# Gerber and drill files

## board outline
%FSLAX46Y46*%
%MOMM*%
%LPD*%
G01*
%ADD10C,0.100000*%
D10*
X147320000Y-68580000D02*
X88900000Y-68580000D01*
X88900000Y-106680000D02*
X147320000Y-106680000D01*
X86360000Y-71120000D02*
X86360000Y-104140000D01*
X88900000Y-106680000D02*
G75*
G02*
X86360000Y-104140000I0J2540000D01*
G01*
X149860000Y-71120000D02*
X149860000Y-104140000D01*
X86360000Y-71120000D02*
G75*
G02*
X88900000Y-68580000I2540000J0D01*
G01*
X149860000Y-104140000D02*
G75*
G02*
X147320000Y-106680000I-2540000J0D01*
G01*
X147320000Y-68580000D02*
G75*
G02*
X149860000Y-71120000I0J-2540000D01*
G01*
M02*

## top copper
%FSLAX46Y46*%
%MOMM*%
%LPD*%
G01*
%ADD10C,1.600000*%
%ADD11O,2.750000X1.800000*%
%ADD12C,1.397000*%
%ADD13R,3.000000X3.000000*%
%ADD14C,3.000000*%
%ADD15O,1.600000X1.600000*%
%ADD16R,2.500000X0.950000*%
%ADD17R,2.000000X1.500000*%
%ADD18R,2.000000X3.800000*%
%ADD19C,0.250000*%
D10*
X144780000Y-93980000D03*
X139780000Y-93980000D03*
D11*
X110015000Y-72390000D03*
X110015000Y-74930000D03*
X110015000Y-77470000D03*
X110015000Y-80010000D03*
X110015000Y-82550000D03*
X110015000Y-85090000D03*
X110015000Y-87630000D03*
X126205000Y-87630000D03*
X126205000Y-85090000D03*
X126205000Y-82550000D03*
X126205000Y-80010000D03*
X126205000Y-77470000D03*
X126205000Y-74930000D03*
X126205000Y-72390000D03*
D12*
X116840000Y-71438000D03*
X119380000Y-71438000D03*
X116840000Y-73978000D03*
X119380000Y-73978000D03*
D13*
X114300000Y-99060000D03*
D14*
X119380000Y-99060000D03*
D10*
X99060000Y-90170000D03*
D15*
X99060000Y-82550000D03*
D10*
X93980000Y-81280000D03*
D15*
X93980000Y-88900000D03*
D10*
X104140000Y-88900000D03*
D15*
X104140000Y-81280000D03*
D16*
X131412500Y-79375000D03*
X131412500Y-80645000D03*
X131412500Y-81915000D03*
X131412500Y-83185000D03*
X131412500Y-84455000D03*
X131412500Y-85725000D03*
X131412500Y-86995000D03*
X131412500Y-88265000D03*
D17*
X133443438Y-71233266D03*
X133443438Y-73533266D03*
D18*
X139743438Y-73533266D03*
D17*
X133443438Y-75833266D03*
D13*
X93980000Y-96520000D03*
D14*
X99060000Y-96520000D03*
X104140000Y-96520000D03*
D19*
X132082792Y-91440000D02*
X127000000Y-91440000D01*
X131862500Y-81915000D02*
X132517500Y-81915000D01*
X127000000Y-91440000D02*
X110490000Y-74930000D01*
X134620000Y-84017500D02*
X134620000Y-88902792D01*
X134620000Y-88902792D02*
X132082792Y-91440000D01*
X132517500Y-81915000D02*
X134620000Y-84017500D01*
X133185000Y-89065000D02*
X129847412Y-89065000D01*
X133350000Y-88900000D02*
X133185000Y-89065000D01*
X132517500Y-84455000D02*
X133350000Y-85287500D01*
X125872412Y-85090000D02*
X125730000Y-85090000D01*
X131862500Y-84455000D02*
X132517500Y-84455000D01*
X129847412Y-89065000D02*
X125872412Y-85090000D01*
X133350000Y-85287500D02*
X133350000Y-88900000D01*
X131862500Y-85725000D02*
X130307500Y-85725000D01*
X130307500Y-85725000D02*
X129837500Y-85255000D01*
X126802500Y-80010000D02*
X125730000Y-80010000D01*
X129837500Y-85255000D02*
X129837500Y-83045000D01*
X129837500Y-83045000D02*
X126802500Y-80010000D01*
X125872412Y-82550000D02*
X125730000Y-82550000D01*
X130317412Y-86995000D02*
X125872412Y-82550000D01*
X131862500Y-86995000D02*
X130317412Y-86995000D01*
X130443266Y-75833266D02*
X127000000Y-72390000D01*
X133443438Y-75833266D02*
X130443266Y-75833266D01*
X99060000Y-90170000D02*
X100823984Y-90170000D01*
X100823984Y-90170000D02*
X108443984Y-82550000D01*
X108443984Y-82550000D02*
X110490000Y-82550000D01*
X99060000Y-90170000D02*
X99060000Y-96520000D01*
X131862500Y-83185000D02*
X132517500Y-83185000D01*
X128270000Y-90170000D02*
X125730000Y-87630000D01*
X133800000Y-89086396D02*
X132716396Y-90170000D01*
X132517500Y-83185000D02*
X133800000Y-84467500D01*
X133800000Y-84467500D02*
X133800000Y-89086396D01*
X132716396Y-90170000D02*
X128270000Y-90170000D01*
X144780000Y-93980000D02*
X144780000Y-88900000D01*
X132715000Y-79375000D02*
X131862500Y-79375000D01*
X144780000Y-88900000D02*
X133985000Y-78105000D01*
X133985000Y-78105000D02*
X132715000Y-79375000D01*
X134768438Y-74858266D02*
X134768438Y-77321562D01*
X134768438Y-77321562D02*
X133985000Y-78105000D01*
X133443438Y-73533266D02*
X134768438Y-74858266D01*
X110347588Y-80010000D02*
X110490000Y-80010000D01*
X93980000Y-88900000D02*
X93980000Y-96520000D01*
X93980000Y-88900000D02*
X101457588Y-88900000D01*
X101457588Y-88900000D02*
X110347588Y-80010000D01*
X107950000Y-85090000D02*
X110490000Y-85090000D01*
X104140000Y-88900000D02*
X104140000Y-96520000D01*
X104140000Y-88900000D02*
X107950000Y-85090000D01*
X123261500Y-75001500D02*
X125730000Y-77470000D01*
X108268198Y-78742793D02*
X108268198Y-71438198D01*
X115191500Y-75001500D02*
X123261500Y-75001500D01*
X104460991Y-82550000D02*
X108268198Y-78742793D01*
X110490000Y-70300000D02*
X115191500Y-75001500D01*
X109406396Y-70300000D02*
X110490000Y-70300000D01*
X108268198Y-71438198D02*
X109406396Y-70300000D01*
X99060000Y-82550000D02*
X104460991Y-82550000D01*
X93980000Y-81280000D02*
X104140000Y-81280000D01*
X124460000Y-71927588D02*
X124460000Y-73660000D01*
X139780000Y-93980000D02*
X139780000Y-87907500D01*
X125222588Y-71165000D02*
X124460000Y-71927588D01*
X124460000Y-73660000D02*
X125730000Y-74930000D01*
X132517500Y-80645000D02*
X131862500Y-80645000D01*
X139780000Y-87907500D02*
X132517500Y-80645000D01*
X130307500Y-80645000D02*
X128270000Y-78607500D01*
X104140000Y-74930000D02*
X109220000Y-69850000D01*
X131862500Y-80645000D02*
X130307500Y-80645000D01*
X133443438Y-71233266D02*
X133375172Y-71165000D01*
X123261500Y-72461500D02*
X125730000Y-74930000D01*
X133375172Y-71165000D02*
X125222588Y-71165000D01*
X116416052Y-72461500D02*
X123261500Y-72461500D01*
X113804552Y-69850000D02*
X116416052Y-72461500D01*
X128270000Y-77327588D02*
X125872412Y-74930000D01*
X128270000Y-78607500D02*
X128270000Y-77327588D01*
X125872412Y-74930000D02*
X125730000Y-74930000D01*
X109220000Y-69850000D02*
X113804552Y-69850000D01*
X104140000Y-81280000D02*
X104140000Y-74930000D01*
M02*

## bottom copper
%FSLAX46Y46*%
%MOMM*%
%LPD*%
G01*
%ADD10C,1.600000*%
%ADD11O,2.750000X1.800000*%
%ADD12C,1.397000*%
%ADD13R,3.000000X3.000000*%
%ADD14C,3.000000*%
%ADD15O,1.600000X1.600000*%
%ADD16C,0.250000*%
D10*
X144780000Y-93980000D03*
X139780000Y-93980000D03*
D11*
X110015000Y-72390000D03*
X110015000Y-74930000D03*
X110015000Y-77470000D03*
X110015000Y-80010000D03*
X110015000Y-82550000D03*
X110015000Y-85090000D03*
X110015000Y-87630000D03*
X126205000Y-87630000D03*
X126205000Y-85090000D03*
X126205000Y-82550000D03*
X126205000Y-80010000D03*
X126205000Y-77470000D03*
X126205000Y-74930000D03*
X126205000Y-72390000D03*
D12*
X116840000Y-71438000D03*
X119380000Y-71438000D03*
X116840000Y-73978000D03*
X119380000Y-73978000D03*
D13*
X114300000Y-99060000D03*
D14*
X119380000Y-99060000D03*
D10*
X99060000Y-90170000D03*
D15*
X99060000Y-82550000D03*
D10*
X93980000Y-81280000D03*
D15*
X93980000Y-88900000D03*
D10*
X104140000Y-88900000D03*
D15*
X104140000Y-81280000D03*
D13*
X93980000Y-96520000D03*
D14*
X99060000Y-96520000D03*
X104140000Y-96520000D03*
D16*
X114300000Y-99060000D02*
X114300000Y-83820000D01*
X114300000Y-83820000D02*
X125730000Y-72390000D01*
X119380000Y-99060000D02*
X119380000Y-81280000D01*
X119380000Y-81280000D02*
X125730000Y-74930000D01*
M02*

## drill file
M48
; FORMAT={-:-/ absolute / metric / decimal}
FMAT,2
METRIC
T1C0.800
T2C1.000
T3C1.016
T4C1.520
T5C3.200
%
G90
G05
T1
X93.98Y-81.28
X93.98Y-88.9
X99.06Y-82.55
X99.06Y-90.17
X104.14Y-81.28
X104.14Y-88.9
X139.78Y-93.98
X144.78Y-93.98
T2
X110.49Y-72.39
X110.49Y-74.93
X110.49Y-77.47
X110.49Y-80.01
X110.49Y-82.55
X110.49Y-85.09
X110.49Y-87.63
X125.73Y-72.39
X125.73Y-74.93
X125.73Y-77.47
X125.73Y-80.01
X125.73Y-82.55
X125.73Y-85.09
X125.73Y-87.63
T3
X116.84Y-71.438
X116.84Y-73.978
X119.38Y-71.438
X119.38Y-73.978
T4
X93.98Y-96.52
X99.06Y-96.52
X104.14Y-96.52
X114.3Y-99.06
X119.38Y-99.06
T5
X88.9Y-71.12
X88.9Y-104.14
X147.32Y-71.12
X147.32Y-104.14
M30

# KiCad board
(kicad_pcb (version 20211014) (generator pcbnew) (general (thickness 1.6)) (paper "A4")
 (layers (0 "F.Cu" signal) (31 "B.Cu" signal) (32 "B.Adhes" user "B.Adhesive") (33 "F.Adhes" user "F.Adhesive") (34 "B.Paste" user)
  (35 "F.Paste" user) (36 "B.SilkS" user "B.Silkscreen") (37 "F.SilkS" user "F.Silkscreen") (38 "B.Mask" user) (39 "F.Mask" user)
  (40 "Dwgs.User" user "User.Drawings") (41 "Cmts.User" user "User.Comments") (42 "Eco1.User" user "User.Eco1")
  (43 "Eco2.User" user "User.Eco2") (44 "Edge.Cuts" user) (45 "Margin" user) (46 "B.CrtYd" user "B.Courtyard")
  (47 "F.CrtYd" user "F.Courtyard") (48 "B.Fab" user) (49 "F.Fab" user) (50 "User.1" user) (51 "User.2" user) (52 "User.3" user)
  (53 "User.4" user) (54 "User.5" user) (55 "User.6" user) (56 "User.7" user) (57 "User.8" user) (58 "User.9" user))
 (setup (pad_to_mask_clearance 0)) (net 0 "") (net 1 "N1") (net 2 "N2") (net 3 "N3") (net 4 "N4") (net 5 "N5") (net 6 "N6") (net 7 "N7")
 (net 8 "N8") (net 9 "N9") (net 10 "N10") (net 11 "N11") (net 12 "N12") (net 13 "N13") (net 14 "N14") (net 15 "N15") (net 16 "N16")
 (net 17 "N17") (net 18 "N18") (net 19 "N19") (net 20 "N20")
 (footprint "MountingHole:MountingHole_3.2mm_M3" (layer "F.Cu") (at 147.32 104.14)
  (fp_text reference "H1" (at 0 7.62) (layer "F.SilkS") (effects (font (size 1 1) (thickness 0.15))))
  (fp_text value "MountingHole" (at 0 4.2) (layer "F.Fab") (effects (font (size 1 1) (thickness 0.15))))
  (pad "" np_thru_hole circle (at 0 0) (size 3.2 3.2) (drill 3.2) (layers *.Cu *.Mask)))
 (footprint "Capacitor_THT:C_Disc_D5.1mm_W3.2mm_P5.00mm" (layer "F.Cu") (at 144.78 93.98 180)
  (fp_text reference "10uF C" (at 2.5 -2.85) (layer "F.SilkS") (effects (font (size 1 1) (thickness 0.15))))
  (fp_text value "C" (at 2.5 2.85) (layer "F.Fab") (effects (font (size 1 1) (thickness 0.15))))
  (pad "1" thru_hole circle (at 0 0 180) (size 1.6 1.6) (drill 0.8) (layers *.Cu *.Mask) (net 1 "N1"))
  (pad "2" thru_hole circle (at 5 0 180) (size 1.6 1.6) (drill 0.8) (layers *.Cu *.Mask) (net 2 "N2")))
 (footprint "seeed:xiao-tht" (layer "F.Cu") (at 118.11 80.01)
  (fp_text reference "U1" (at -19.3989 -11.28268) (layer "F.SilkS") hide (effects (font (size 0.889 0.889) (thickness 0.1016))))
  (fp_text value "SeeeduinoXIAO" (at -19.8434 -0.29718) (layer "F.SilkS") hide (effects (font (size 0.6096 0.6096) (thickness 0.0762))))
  (pad "1" thru_hole oval (at -7.62 -7.62) (size 2.75 1.8) (drill 1 (offset -0.475 0)) (layers *.Cu *.Mask) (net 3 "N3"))
  (pad "2" thru_hole oval (at -7.62 -5.08) (size 2.75 1.8) (drill 1 (offset -0.475 0)) (layers *.Cu *.Mask) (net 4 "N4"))
  (pad "3" thru_hole oval (at -7.62 -2.54) (size 2.75 1.8) (drill 1 (offset -0.475 0)) (layers *.Cu *.Mask) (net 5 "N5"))
  (pad "4" thru_hole oval (at -7.62 0) (size 2.75 1.8) (drill 1 (offset -0.475 0)) (layers *.Cu *.Mask) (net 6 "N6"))
  (pad "5" thru_hole oval (at -7.62 2.54) (size 2.75 1.8) (drill 1 (offset -0.475 0)) (layers *.Cu *.Mask) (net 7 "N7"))
  (pad "6" thru_hole oval (at -7.62 5.08) (size 2.75 1.8) (drill 1 (offset -0.475 0)) (layers *.Cu *.Mask) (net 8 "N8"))
  (pad "7" thru_hole oval (at -7.62 7.62) (size 2.75 1.8) (drill 1 (offset -0.475 0)) (layers *.Cu *.Mask) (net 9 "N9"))
  (pad "8" thru_hole oval (at 7.62 7.62 180) (size 2.75 1.8) (drill 1 (offset -0.475 0)) (layers *.Cu *.Mask) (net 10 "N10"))
  (pad "9" thru_hole oval (at 7.62 5.08 180) (size 2.75 1.8) (drill 1 (offset -0.475 0)) (layers *.Cu *.Mask) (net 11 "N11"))
  (pad "10" thru_hole oval (at 7.62 2.54 180) (size 2.75 1.8) (drill 1 (offset -0.475 0)) (layers *.Cu *.Mask) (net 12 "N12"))
  (pad "11" thru_hole oval (at 7.62 0 180) (size 2.75 1.8) (drill 1 (offset -0.475 0)) (layers *.Cu *.Mask) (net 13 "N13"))
  (pad "12" thru_hole oval (at 7.62 -2.54 180) (size 2.75 1.8) (drill 1 (offset -0.475 0)) (layers *.Cu *.Mask) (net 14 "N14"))
  (pad "13" thru_hole oval (at 7.62 -5.08 180) (size 2.75 1.8) (drill 1 (offset -0.475 0)) (layers *.Cu *.Mask) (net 2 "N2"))
  (pad "14" thru_hole oval (at 7.62 -7.62 180) (size 2.75 1.8) (drill 1 (offset -0.475 0)) (layers *.Cu *.Mask) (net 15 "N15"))
  (pad "15" thru_hole circle (at -1.27 -8.572 90) (size 1.397 1.397) (drill 1.016) (layers *.Cu *.Mask) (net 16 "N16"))
  (pad "16" thru_hole circle (at 1.27 -8.572 90) (size 1.397 1.397) (drill 1.016) (layers *.Cu *.Mask) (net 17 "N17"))
  (pad "17" thru_hole circle (at -1.27 -6.032 90) (size 1.397 1.397) (drill 1.016) (layers *.Cu *.Mask) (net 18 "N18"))
  (pad "18" thru_hole circle (at 1.27 -6.032 90) (size 1.397 1.397) (drill 1.016) (layers *.Cu *.Mask) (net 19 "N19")))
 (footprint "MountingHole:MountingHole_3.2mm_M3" (layer "F.Cu") (at 88.9 104.14)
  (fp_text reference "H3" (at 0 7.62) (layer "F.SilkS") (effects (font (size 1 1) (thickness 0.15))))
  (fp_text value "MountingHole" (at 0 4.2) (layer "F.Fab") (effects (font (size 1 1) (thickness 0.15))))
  (pad "" np_thru_hole circle (at 0 0) (size 3.2 3.2) (drill 3.2) (layers *.Cu *.Mask)))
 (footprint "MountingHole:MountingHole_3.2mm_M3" (layer "F.Cu") (at 147.32 71.12)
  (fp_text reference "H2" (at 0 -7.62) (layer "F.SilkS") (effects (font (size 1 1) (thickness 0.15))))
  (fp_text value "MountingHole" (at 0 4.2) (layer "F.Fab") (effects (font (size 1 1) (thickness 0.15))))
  (pad "" np_thru_hole circle (at 0 0) (size 3.2 3.2) (drill 3.2) (layers *.Cu *.Mask)))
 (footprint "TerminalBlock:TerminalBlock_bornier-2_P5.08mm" (layer "F.Cu") (at 114.3 99.06)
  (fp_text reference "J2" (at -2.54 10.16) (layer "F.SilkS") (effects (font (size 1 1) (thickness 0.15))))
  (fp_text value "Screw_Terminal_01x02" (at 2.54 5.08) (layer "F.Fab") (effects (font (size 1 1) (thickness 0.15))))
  (pad "1" thru_hole rect (at 0 0) (size 3 3) (drill 1.52) (layers *.Cu *.Mask) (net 15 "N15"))
  (pad "2" thru_hole circle (at 5.08 0) (size 3 3) (drill 1.52) (layers *.Cu *.Mask) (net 2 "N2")))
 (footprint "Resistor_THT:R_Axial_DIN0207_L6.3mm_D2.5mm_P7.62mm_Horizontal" (layer "F.Cu") (at 99.06 90.17 90)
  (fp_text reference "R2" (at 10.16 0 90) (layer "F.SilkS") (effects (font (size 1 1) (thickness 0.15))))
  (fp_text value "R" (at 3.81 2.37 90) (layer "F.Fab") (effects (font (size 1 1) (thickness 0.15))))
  (pad "1" thru_hole circle (at 0 0 90) (size 1.6 1.6) (drill 0.8) (layers *.Cu *.Mask) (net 7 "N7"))
  (pad "2" thru_hole oval (at 7.62 0 90) (size 1.6 1.6) (drill 0.8) (layers *.Cu *.Mask) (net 14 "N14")))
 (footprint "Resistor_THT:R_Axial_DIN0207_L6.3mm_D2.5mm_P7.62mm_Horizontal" (layer "F.Cu") (at 93.98 81.28 -90)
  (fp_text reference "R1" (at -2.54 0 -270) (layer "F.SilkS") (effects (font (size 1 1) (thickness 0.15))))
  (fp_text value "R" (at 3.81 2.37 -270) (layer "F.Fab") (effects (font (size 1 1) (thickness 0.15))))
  (pad "1" thru_hole circle (at 0 0 270) (size 1.6 1.6) (drill 0.8) (layers *.Cu *.Mask) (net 2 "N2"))
  (pad "2" thru_hole oval (at 7.62 0 270) (size 1.6 1.6) (drill 0.8) (layers *.Cu *.Mask) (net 6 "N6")))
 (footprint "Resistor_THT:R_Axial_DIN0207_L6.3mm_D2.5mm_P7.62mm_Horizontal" (layer "F.Cu") (at 104.14 88.9 90)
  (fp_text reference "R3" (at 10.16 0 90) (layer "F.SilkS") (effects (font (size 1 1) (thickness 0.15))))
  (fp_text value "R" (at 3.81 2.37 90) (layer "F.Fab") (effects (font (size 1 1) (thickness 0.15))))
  (pad "1" thru_hole circle (at 0 0 90) (size 1.6 1.6) (drill 0.8) (layers *.Cu *.Mask) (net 8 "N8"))
  (pad "2" thru_hole oval (at 7.62 0 90) (size 1.6 1.6) (drill 0.8) (layers *.Cu *.Mask) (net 2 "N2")))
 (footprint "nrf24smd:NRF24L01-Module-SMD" (layer "F.Cu") (at 132.1625 83.82 180)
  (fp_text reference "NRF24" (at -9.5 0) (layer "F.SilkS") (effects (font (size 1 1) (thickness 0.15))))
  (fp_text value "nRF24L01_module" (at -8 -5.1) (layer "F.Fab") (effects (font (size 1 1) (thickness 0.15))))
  (pad "1" smd rect locked (at 0.3 4.445 180) (size 2.5 0.95) (drill (offset 0.45 0)) (layers "F.Cu" "F.Paste" "F.Mask") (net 1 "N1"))
  (pad "2" smd rect locked (at 0.3 3.175 180) (size 2.5 0.95) (drill (offset 0.45 0)) (layers "F.Cu" "F.Paste" "F.Mask") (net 2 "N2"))
  (pad "3" smd rect (at 0.3 1.905 180) (size 2.5 0.95) (drill (offset 0.45 0)) (layers "F.Cu" "F.Paste" "F.Mask") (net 4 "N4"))
  (pad "4" smd rect locked (at 0.3 0.635 180) (size 2.5 0.95) (drill (offset 0.45 0)) (layers "F.Cu" "F.Paste" "F.Mask") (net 10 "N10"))
  (pad "5" smd rect locked (at 0.3 -0.635 180) (size 2.5 0.95) (drill (offset 0.45 0)) (layers "F.Cu" "F.Paste" "F.Mask") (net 11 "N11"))
  (pad "6" smd rect locked (at 0.3 -1.905 180) (size 2.5 0.95) (drill (offset 0.45 0)) (layers "F.Cu" "F.Paste" "F.Mask") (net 13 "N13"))
  (pad "7" smd rect locked (at 0.3 -3.175 180) (size 2.5 0.95) (drill (offset 0.45 0)) (layers "F.Cu" "F.Paste" "F.Mask") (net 12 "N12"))
  (pad "8" smd rect locked (at 0.3 -4.445 180) (size 2.5 0.95) (drill (offset 0.45 0)) (layers "F.Cu" "F.Paste" "F.Mask") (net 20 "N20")))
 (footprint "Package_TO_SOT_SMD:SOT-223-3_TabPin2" (layer "F.Cu") (at 136.593438 73.533266)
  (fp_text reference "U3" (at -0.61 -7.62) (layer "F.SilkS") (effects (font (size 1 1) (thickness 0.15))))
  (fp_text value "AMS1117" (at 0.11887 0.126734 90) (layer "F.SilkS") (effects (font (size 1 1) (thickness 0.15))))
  (pad "1" smd rect (at -3.15 -2.3) (size 2 1.5) (layers "F.Cu" "F.Paste" "F.Mask") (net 2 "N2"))
  (pad "2" smd rect (at -3.15 0) (size 2 1.5) (layers "F.Cu" "F.Paste" "F.Mask") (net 1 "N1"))
  (pad "2" smd rect (at 3.15 0) (size 2 3.8) (layers "F.Cu" "F.Paste" "F.Mask") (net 1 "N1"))
  (pad "3" smd rect (at -3.15 2.3) (size 2 1.5) (layers "F.Cu" "F.Paste" "F.Mask") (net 15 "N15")))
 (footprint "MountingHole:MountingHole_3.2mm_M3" (layer "F.Cu") (at 88.9 71.12)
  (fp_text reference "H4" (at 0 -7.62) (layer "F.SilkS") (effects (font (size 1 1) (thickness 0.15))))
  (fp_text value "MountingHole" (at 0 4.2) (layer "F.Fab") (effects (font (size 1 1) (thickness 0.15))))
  (pad "" np_thru_hole circle (at 0 0) (size 3.2 3.2) (drill 3.2) (layers *.Cu *.Mask)))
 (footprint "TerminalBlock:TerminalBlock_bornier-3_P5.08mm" (layer "F.Cu") (at 93.98 96.52)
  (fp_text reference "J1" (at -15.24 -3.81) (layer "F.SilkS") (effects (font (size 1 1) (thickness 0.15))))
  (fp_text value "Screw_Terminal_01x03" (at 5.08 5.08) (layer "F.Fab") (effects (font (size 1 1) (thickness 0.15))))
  (pad "1" thru_hole rect (at 0 0) (size 3 3) (drill 1.52) (layers *.Cu *.Mask) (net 6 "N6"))
  (pad "2" thru_hole circle (at 5.08 0) (size 3 3) (drill 1.52) (layers *.Cu *.Mask) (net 7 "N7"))
  (pad "3" thru_hole circle (at 10.16 0) (size 3 3) (drill 1.52) (layers *.Cu *.Mask) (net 8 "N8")))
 (gr_line (start 147.32 68.58) (end 88.9 68.58) (layer "Edge.Cuts") (width 0.1))
 (gr_line (start 88.9 106.68) (end 147.32 106.68) (layer "Edge.Cuts") (width 0.1))
 (gr_line (start 86.36 71.12) (end 86.36 104.14) (layer "Edge.Cuts") (width 0.1))
 (gr_arc (start 88.9 106.68) (mid 87.103949 105.936051) (end 86.36 104.14) (layer "Edge.Cuts") (width 0.1))
 (gr_line (start 149.86 71.12) (end 149.86 104.14) (layer "Edge.Cuts") (width 0.1))
 (gr_arc (start 86.36 71.12) (mid 87.103949 69.323949) (end 88.9 68.58) (layer "Edge.Cuts") (width 0.1))
 (gr_arc (start 149.86 104.14) (mid 149.116051 105.936051) (end 147.32 106.68) (layer "Edge.Cuts") (width 0.1))
 (gr_arc (start 147.32 68.58) (mid 149.116051 69.323949) (end 149.86 71.12) (layer "Edge.Cuts") (width 0.1))
 (segment (start 132.082792 91.44) (end 127 91.44) (width 0.25) (layer "F.Cu") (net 4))
 (segment (start 131.8625 81.915) (end 132.5175 81.915) (width 0.25) (layer "F.Cu") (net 4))
 (segment (start 127 91.44) (end 110.49 74.93) (width 0.25) (layer "F.Cu") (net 4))
 (segment (start 134.62 84.0175) (end 134.62 88.902792) (width 0.25) (layer "F.Cu") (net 4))
 (segment (start 134.62 88.902792) (end 132.082792 91.44) (width 0.25) (layer "F.Cu") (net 4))
 (segment (start 132.5175 81.915) (end 134.62 84.0175) (width 0.25) (layer "F.Cu") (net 4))
 (segment (start 133.185 89.065) (end 129.847412 89.065) (width 0.25) (layer "F.Cu") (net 11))
 (segment (start 133.35 88.9) (end 133.185 89.065) (width 0.25) (layer "F.Cu") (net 11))
 (segment (start 132.5175 84.455) (end 133.35 85.2875) (width 0.25) (layer "F.Cu") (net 11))
 (segment (start 125.872412 85.09) (end 125.73 85.09) (width 0.25) (layer "F.Cu") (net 11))
 (segment (start 131.8625 84.455) (end 132.5175 84.455) (width 0.25) (layer "F.Cu") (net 11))
 (segment (start 129.847412 89.065) (end 125.872412 85.09) (width 0.25) (layer "F.Cu") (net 11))
 (segment (start 133.35 85.2875) (end 133.35 88.9) (width 0.25) (layer "F.Cu") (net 11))
 (segment (start 131.8625 85.725) (end 130.3075 85.725) (width 0.25) (layer "F.Cu") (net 13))
 (segment (start 130.3075 85.725) (end 129.8375 85.255) (width 0.25) (layer "F.Cu") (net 13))
 (segment (start 126.8025 80.01) (end 125.73 80.01) (width 0.25) (layer "F.Cu") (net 13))
 (segment (start 129.8375 85.255) (end 129.8375 83.045) (width 0.25) (layer "F.Cu") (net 13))
 (segment (start 129.8375 83.045) (end 126.8025 80.01) (width 0.25) (layer "F.Cu") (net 13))
 (segment (start 125.872412 82.55) (end 125.73 82.55) (width 0.25) (layer "F.Cu") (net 12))
 (segment (start 130.317412 86.995) (end 125.872412 82.55) (width 0.25) (layer "F.Cu") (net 12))
 (segment (start 131.8625 86.995) (end 130.317412 86.995) (width 0.25) (layer "F.Cu") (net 12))
 (segment (start 130.443266 75.833266) (end 127 72.39) (width 0.25) (layer "F.Cu") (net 15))
 (segment (start 133.443438 75.833266) (end 130.443266 75.833266) (width 0.25) (layer "F.Cu") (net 15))
 (segment (start 114.3 99.06) (end 114.3 83.82) (width 0.25) (layer "B.Cu") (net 15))
 (segment (start 114.3 83.82) (end 125.73 72.39) (width 0.25) (layer "B.Cu") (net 15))
 (segment (start 99.06 90.17) (end 100.823984 90.17) (width 0.25) (layer "F.Cu") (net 7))
 (segment (start 100.823984 90.17) (end 108.443984 82.55) (width 0.25) (layer "F.Cu") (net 7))
 (segment (start 108.443984 82.55) (end 110.49 82.55) (width 0.25) (layer "F.Cu") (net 7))
 (segment (start 99.06 90.17) (end 99.06 96.52) (width 0.25) (layer "F.Cu") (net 7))
 (segment (start 131.8625 83.185) (end 132.5175 83.185) (width 0.25) (layer "F.Cu") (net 10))
 (segment (start 128.27 90.17) (end 125.73 87.63) (width 0.25) (layer "F.Cu") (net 10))
 (segment (start 133.8 89.086396) (end 132.716396 90.17) (width 0.25) (layer "F.Cu") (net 10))
 (segment (start 132.5175 83.185) (end 133.8 84.4675) (width 0.25) (layer "F.Cu") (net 10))
 (segment (start 133.8 84.4675) (end 133.8 89.086396) (width 0.25) (layer "F.Cu") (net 10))
 (segment (start 132.716396 90.17) (end 128.27 90.17) (width 0.25) (layer "F.Cu") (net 10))
 (segment (start 144.78 93.98) (end 144.78 88.9) (width 0.25) (layer "F.Cu") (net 1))
 (segment (start 132.715 79.375) (end 131.8625 79.375) (width 0.25) (layer "F.Cu") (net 1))
 (segment (start 144.78 88.9) (end 133.985 78.105) (width 0.25) (layer "F.Cu") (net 1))
 (segment (start 133.985 78.105) (end 132.715 79.375) (width 0.25) (layer "F.Cu") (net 1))
 (segment (start 134.768438 74.858266) (end 134.768438 77.321562) (width 0.25) (layer "F.Cu") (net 1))
 (segment (start 134.768438 77.321562) (end 133.985 78.105) (width 0.25) (layer "F.Cu") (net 1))
 (segment (start 133.443438 73.533266) (end 134.768438 74.858266) (width 0.25) (layer "F.Cu") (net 1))
 (segment (start 110.347588 80.01) (end 110.49 80.01) (width 0.25) (layer "F.Cu") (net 6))
 (segment (start 93.98 88.9) (end 93.98 96.52) (width 0.25) (layer "F.Cu") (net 6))
 (segment (start 93.98 88.9) (end 101.457588 88.9) (width 0.25) (layer "F.Cu") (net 6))
 (segment (start 101.457588 88.9) (end 110.347588 80.01) (width 0.25) (layer "F.Cu") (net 6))
 (segment (start 107.95 85.09) (end 110.49 85.09) (width 0.25) (layer "F.Cu") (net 8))
 (segment (start 104.14 88.9) (end 104.14 96.52) (width 0.25) (layer "F.Cu") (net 8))
 (segment (start 104.14 88.9) (end 107.95 85.09) (width 0.25) (layer "F.Cu") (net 8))
 (segment (start 123.2615 75.0015) (end 125.73 77.47) (width 0.25) (layer "F.Cu") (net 14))
 (segment (start 108.268198 78.742793) (end 108.268198 71.438198) (width 0.25) (layer "F.Cu") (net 14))
 (segment (start 115.1915 75.0015) (end 123.2615 75.0015) (width 0.25) (layer "F.Cu") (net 14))
 (segment (start 104.460991 82.55) (end 108.268198 78.742793) (width 0.25) (layer "F.Cu") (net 14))
 (segment (start 110.49 70.3) (end 115.1915 75.0015) (width 0.25) (layer "F.Cu") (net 14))
 (segment (start 109.406396 70.3) (end 110.49 70.3) (width 0.25) (layer "F.Cu") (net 14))
 (segment (start 108.268198 71.438198) (end 109.406396 70.3) (width 0.25) (layer "F.Cu") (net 14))
 (segment (start 99.06 82.55) (end 104.460991 82.55) (width 0.25) (layer "F.Cu") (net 14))
 (segment (start 93.98 81.28) (end 104.14 81.28) (width 0.25) (layer "F.Cu") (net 2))
 (segment (start 124.46 71.927588) (end 124.46 73.66) (width 0.25) (layer "F.Cu") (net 2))
 (segment (start 139.78 93.98) (end 139.78 87.9075) (width 0.25) (layer "F.Cu") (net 2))
 (segment (start 125.222588 71.165) (end 124.46 71.927588) (width 0.25) (layer "F.Cu") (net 2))
 (segment (start 124.46 73.66) (end 125.73 74.93) (width 0.25) (layer "F.Cu") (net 2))
 (segment (start 132.5175 80.645) (end 131.8625 80.645) (width 0.25) (layer "F.Cu") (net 2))
 (segment (start 139.78 87.9075) (end 132.5175 80.645) (width 0.25) (layer "F.Cu") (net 2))
 (segment (start 130.3075 80.645) (end 128.27 78.6075) (width 0.25) (layer "F.Cu") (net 2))
 (segment (start 104.14 74.93) (end 109.22 69.85) (width 0.25) (layer "F.Cu") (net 2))
 (segment (start 131.8625 80.645) (end 130.3075 80.645) (width 0.25) (layer "F.Cu") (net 2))
 (segment (start 133.443438 71.233266) (end 133.375172 71.165) (width 0.25) (layer "F.Cu") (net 2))
 (segment (start 123.2615 72.4615) (end 125.73 74.93) (width 0.25) (layer "F.Cu") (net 2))
 (segment (start 133.375172 71.165) (end 125.222588 71.165) (width 0.25) (layer "F.Cu") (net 2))
 (segment (start 116.416052 72.4615) (end 123.2615 72.4615) (width 0.25) (layer "F.Cu") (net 2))
 (segment (start 113.804552 69.85) (end 116.416052 72.4615) (width 0.25) (layer "F.Cu") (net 2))
 (segment (start 128.27 77.327588) (end 125.872412 74.93) (width 0.25) (layer "F.Cu") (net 2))
 (segment (start 128.27 78.6075) (end 128.27 77.327588) (width 0.25) (layer "F.Cu") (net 2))
 (segment (start 125.872412 74.93) (end 125.73 74.93) (width 0.25) (layer "F.Cu") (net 2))
 (segment (start 109.22 69.85) (end 113.804552 69.85) (width 0.25) (layer "F.Cu") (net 2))
 (segment (start 104.14 81.28) (end 104.14 74.93) (width 0.25) (layer "F.Cu") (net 2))
 (segment (start 119.38 99.06) (end 119.38 81.28) (width 0.25) (layer "B.Cu") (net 2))
 (segment (start 119.38 81.28) (end 125.73 74.93) (width 0.25) (layer "B.Cu") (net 2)))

